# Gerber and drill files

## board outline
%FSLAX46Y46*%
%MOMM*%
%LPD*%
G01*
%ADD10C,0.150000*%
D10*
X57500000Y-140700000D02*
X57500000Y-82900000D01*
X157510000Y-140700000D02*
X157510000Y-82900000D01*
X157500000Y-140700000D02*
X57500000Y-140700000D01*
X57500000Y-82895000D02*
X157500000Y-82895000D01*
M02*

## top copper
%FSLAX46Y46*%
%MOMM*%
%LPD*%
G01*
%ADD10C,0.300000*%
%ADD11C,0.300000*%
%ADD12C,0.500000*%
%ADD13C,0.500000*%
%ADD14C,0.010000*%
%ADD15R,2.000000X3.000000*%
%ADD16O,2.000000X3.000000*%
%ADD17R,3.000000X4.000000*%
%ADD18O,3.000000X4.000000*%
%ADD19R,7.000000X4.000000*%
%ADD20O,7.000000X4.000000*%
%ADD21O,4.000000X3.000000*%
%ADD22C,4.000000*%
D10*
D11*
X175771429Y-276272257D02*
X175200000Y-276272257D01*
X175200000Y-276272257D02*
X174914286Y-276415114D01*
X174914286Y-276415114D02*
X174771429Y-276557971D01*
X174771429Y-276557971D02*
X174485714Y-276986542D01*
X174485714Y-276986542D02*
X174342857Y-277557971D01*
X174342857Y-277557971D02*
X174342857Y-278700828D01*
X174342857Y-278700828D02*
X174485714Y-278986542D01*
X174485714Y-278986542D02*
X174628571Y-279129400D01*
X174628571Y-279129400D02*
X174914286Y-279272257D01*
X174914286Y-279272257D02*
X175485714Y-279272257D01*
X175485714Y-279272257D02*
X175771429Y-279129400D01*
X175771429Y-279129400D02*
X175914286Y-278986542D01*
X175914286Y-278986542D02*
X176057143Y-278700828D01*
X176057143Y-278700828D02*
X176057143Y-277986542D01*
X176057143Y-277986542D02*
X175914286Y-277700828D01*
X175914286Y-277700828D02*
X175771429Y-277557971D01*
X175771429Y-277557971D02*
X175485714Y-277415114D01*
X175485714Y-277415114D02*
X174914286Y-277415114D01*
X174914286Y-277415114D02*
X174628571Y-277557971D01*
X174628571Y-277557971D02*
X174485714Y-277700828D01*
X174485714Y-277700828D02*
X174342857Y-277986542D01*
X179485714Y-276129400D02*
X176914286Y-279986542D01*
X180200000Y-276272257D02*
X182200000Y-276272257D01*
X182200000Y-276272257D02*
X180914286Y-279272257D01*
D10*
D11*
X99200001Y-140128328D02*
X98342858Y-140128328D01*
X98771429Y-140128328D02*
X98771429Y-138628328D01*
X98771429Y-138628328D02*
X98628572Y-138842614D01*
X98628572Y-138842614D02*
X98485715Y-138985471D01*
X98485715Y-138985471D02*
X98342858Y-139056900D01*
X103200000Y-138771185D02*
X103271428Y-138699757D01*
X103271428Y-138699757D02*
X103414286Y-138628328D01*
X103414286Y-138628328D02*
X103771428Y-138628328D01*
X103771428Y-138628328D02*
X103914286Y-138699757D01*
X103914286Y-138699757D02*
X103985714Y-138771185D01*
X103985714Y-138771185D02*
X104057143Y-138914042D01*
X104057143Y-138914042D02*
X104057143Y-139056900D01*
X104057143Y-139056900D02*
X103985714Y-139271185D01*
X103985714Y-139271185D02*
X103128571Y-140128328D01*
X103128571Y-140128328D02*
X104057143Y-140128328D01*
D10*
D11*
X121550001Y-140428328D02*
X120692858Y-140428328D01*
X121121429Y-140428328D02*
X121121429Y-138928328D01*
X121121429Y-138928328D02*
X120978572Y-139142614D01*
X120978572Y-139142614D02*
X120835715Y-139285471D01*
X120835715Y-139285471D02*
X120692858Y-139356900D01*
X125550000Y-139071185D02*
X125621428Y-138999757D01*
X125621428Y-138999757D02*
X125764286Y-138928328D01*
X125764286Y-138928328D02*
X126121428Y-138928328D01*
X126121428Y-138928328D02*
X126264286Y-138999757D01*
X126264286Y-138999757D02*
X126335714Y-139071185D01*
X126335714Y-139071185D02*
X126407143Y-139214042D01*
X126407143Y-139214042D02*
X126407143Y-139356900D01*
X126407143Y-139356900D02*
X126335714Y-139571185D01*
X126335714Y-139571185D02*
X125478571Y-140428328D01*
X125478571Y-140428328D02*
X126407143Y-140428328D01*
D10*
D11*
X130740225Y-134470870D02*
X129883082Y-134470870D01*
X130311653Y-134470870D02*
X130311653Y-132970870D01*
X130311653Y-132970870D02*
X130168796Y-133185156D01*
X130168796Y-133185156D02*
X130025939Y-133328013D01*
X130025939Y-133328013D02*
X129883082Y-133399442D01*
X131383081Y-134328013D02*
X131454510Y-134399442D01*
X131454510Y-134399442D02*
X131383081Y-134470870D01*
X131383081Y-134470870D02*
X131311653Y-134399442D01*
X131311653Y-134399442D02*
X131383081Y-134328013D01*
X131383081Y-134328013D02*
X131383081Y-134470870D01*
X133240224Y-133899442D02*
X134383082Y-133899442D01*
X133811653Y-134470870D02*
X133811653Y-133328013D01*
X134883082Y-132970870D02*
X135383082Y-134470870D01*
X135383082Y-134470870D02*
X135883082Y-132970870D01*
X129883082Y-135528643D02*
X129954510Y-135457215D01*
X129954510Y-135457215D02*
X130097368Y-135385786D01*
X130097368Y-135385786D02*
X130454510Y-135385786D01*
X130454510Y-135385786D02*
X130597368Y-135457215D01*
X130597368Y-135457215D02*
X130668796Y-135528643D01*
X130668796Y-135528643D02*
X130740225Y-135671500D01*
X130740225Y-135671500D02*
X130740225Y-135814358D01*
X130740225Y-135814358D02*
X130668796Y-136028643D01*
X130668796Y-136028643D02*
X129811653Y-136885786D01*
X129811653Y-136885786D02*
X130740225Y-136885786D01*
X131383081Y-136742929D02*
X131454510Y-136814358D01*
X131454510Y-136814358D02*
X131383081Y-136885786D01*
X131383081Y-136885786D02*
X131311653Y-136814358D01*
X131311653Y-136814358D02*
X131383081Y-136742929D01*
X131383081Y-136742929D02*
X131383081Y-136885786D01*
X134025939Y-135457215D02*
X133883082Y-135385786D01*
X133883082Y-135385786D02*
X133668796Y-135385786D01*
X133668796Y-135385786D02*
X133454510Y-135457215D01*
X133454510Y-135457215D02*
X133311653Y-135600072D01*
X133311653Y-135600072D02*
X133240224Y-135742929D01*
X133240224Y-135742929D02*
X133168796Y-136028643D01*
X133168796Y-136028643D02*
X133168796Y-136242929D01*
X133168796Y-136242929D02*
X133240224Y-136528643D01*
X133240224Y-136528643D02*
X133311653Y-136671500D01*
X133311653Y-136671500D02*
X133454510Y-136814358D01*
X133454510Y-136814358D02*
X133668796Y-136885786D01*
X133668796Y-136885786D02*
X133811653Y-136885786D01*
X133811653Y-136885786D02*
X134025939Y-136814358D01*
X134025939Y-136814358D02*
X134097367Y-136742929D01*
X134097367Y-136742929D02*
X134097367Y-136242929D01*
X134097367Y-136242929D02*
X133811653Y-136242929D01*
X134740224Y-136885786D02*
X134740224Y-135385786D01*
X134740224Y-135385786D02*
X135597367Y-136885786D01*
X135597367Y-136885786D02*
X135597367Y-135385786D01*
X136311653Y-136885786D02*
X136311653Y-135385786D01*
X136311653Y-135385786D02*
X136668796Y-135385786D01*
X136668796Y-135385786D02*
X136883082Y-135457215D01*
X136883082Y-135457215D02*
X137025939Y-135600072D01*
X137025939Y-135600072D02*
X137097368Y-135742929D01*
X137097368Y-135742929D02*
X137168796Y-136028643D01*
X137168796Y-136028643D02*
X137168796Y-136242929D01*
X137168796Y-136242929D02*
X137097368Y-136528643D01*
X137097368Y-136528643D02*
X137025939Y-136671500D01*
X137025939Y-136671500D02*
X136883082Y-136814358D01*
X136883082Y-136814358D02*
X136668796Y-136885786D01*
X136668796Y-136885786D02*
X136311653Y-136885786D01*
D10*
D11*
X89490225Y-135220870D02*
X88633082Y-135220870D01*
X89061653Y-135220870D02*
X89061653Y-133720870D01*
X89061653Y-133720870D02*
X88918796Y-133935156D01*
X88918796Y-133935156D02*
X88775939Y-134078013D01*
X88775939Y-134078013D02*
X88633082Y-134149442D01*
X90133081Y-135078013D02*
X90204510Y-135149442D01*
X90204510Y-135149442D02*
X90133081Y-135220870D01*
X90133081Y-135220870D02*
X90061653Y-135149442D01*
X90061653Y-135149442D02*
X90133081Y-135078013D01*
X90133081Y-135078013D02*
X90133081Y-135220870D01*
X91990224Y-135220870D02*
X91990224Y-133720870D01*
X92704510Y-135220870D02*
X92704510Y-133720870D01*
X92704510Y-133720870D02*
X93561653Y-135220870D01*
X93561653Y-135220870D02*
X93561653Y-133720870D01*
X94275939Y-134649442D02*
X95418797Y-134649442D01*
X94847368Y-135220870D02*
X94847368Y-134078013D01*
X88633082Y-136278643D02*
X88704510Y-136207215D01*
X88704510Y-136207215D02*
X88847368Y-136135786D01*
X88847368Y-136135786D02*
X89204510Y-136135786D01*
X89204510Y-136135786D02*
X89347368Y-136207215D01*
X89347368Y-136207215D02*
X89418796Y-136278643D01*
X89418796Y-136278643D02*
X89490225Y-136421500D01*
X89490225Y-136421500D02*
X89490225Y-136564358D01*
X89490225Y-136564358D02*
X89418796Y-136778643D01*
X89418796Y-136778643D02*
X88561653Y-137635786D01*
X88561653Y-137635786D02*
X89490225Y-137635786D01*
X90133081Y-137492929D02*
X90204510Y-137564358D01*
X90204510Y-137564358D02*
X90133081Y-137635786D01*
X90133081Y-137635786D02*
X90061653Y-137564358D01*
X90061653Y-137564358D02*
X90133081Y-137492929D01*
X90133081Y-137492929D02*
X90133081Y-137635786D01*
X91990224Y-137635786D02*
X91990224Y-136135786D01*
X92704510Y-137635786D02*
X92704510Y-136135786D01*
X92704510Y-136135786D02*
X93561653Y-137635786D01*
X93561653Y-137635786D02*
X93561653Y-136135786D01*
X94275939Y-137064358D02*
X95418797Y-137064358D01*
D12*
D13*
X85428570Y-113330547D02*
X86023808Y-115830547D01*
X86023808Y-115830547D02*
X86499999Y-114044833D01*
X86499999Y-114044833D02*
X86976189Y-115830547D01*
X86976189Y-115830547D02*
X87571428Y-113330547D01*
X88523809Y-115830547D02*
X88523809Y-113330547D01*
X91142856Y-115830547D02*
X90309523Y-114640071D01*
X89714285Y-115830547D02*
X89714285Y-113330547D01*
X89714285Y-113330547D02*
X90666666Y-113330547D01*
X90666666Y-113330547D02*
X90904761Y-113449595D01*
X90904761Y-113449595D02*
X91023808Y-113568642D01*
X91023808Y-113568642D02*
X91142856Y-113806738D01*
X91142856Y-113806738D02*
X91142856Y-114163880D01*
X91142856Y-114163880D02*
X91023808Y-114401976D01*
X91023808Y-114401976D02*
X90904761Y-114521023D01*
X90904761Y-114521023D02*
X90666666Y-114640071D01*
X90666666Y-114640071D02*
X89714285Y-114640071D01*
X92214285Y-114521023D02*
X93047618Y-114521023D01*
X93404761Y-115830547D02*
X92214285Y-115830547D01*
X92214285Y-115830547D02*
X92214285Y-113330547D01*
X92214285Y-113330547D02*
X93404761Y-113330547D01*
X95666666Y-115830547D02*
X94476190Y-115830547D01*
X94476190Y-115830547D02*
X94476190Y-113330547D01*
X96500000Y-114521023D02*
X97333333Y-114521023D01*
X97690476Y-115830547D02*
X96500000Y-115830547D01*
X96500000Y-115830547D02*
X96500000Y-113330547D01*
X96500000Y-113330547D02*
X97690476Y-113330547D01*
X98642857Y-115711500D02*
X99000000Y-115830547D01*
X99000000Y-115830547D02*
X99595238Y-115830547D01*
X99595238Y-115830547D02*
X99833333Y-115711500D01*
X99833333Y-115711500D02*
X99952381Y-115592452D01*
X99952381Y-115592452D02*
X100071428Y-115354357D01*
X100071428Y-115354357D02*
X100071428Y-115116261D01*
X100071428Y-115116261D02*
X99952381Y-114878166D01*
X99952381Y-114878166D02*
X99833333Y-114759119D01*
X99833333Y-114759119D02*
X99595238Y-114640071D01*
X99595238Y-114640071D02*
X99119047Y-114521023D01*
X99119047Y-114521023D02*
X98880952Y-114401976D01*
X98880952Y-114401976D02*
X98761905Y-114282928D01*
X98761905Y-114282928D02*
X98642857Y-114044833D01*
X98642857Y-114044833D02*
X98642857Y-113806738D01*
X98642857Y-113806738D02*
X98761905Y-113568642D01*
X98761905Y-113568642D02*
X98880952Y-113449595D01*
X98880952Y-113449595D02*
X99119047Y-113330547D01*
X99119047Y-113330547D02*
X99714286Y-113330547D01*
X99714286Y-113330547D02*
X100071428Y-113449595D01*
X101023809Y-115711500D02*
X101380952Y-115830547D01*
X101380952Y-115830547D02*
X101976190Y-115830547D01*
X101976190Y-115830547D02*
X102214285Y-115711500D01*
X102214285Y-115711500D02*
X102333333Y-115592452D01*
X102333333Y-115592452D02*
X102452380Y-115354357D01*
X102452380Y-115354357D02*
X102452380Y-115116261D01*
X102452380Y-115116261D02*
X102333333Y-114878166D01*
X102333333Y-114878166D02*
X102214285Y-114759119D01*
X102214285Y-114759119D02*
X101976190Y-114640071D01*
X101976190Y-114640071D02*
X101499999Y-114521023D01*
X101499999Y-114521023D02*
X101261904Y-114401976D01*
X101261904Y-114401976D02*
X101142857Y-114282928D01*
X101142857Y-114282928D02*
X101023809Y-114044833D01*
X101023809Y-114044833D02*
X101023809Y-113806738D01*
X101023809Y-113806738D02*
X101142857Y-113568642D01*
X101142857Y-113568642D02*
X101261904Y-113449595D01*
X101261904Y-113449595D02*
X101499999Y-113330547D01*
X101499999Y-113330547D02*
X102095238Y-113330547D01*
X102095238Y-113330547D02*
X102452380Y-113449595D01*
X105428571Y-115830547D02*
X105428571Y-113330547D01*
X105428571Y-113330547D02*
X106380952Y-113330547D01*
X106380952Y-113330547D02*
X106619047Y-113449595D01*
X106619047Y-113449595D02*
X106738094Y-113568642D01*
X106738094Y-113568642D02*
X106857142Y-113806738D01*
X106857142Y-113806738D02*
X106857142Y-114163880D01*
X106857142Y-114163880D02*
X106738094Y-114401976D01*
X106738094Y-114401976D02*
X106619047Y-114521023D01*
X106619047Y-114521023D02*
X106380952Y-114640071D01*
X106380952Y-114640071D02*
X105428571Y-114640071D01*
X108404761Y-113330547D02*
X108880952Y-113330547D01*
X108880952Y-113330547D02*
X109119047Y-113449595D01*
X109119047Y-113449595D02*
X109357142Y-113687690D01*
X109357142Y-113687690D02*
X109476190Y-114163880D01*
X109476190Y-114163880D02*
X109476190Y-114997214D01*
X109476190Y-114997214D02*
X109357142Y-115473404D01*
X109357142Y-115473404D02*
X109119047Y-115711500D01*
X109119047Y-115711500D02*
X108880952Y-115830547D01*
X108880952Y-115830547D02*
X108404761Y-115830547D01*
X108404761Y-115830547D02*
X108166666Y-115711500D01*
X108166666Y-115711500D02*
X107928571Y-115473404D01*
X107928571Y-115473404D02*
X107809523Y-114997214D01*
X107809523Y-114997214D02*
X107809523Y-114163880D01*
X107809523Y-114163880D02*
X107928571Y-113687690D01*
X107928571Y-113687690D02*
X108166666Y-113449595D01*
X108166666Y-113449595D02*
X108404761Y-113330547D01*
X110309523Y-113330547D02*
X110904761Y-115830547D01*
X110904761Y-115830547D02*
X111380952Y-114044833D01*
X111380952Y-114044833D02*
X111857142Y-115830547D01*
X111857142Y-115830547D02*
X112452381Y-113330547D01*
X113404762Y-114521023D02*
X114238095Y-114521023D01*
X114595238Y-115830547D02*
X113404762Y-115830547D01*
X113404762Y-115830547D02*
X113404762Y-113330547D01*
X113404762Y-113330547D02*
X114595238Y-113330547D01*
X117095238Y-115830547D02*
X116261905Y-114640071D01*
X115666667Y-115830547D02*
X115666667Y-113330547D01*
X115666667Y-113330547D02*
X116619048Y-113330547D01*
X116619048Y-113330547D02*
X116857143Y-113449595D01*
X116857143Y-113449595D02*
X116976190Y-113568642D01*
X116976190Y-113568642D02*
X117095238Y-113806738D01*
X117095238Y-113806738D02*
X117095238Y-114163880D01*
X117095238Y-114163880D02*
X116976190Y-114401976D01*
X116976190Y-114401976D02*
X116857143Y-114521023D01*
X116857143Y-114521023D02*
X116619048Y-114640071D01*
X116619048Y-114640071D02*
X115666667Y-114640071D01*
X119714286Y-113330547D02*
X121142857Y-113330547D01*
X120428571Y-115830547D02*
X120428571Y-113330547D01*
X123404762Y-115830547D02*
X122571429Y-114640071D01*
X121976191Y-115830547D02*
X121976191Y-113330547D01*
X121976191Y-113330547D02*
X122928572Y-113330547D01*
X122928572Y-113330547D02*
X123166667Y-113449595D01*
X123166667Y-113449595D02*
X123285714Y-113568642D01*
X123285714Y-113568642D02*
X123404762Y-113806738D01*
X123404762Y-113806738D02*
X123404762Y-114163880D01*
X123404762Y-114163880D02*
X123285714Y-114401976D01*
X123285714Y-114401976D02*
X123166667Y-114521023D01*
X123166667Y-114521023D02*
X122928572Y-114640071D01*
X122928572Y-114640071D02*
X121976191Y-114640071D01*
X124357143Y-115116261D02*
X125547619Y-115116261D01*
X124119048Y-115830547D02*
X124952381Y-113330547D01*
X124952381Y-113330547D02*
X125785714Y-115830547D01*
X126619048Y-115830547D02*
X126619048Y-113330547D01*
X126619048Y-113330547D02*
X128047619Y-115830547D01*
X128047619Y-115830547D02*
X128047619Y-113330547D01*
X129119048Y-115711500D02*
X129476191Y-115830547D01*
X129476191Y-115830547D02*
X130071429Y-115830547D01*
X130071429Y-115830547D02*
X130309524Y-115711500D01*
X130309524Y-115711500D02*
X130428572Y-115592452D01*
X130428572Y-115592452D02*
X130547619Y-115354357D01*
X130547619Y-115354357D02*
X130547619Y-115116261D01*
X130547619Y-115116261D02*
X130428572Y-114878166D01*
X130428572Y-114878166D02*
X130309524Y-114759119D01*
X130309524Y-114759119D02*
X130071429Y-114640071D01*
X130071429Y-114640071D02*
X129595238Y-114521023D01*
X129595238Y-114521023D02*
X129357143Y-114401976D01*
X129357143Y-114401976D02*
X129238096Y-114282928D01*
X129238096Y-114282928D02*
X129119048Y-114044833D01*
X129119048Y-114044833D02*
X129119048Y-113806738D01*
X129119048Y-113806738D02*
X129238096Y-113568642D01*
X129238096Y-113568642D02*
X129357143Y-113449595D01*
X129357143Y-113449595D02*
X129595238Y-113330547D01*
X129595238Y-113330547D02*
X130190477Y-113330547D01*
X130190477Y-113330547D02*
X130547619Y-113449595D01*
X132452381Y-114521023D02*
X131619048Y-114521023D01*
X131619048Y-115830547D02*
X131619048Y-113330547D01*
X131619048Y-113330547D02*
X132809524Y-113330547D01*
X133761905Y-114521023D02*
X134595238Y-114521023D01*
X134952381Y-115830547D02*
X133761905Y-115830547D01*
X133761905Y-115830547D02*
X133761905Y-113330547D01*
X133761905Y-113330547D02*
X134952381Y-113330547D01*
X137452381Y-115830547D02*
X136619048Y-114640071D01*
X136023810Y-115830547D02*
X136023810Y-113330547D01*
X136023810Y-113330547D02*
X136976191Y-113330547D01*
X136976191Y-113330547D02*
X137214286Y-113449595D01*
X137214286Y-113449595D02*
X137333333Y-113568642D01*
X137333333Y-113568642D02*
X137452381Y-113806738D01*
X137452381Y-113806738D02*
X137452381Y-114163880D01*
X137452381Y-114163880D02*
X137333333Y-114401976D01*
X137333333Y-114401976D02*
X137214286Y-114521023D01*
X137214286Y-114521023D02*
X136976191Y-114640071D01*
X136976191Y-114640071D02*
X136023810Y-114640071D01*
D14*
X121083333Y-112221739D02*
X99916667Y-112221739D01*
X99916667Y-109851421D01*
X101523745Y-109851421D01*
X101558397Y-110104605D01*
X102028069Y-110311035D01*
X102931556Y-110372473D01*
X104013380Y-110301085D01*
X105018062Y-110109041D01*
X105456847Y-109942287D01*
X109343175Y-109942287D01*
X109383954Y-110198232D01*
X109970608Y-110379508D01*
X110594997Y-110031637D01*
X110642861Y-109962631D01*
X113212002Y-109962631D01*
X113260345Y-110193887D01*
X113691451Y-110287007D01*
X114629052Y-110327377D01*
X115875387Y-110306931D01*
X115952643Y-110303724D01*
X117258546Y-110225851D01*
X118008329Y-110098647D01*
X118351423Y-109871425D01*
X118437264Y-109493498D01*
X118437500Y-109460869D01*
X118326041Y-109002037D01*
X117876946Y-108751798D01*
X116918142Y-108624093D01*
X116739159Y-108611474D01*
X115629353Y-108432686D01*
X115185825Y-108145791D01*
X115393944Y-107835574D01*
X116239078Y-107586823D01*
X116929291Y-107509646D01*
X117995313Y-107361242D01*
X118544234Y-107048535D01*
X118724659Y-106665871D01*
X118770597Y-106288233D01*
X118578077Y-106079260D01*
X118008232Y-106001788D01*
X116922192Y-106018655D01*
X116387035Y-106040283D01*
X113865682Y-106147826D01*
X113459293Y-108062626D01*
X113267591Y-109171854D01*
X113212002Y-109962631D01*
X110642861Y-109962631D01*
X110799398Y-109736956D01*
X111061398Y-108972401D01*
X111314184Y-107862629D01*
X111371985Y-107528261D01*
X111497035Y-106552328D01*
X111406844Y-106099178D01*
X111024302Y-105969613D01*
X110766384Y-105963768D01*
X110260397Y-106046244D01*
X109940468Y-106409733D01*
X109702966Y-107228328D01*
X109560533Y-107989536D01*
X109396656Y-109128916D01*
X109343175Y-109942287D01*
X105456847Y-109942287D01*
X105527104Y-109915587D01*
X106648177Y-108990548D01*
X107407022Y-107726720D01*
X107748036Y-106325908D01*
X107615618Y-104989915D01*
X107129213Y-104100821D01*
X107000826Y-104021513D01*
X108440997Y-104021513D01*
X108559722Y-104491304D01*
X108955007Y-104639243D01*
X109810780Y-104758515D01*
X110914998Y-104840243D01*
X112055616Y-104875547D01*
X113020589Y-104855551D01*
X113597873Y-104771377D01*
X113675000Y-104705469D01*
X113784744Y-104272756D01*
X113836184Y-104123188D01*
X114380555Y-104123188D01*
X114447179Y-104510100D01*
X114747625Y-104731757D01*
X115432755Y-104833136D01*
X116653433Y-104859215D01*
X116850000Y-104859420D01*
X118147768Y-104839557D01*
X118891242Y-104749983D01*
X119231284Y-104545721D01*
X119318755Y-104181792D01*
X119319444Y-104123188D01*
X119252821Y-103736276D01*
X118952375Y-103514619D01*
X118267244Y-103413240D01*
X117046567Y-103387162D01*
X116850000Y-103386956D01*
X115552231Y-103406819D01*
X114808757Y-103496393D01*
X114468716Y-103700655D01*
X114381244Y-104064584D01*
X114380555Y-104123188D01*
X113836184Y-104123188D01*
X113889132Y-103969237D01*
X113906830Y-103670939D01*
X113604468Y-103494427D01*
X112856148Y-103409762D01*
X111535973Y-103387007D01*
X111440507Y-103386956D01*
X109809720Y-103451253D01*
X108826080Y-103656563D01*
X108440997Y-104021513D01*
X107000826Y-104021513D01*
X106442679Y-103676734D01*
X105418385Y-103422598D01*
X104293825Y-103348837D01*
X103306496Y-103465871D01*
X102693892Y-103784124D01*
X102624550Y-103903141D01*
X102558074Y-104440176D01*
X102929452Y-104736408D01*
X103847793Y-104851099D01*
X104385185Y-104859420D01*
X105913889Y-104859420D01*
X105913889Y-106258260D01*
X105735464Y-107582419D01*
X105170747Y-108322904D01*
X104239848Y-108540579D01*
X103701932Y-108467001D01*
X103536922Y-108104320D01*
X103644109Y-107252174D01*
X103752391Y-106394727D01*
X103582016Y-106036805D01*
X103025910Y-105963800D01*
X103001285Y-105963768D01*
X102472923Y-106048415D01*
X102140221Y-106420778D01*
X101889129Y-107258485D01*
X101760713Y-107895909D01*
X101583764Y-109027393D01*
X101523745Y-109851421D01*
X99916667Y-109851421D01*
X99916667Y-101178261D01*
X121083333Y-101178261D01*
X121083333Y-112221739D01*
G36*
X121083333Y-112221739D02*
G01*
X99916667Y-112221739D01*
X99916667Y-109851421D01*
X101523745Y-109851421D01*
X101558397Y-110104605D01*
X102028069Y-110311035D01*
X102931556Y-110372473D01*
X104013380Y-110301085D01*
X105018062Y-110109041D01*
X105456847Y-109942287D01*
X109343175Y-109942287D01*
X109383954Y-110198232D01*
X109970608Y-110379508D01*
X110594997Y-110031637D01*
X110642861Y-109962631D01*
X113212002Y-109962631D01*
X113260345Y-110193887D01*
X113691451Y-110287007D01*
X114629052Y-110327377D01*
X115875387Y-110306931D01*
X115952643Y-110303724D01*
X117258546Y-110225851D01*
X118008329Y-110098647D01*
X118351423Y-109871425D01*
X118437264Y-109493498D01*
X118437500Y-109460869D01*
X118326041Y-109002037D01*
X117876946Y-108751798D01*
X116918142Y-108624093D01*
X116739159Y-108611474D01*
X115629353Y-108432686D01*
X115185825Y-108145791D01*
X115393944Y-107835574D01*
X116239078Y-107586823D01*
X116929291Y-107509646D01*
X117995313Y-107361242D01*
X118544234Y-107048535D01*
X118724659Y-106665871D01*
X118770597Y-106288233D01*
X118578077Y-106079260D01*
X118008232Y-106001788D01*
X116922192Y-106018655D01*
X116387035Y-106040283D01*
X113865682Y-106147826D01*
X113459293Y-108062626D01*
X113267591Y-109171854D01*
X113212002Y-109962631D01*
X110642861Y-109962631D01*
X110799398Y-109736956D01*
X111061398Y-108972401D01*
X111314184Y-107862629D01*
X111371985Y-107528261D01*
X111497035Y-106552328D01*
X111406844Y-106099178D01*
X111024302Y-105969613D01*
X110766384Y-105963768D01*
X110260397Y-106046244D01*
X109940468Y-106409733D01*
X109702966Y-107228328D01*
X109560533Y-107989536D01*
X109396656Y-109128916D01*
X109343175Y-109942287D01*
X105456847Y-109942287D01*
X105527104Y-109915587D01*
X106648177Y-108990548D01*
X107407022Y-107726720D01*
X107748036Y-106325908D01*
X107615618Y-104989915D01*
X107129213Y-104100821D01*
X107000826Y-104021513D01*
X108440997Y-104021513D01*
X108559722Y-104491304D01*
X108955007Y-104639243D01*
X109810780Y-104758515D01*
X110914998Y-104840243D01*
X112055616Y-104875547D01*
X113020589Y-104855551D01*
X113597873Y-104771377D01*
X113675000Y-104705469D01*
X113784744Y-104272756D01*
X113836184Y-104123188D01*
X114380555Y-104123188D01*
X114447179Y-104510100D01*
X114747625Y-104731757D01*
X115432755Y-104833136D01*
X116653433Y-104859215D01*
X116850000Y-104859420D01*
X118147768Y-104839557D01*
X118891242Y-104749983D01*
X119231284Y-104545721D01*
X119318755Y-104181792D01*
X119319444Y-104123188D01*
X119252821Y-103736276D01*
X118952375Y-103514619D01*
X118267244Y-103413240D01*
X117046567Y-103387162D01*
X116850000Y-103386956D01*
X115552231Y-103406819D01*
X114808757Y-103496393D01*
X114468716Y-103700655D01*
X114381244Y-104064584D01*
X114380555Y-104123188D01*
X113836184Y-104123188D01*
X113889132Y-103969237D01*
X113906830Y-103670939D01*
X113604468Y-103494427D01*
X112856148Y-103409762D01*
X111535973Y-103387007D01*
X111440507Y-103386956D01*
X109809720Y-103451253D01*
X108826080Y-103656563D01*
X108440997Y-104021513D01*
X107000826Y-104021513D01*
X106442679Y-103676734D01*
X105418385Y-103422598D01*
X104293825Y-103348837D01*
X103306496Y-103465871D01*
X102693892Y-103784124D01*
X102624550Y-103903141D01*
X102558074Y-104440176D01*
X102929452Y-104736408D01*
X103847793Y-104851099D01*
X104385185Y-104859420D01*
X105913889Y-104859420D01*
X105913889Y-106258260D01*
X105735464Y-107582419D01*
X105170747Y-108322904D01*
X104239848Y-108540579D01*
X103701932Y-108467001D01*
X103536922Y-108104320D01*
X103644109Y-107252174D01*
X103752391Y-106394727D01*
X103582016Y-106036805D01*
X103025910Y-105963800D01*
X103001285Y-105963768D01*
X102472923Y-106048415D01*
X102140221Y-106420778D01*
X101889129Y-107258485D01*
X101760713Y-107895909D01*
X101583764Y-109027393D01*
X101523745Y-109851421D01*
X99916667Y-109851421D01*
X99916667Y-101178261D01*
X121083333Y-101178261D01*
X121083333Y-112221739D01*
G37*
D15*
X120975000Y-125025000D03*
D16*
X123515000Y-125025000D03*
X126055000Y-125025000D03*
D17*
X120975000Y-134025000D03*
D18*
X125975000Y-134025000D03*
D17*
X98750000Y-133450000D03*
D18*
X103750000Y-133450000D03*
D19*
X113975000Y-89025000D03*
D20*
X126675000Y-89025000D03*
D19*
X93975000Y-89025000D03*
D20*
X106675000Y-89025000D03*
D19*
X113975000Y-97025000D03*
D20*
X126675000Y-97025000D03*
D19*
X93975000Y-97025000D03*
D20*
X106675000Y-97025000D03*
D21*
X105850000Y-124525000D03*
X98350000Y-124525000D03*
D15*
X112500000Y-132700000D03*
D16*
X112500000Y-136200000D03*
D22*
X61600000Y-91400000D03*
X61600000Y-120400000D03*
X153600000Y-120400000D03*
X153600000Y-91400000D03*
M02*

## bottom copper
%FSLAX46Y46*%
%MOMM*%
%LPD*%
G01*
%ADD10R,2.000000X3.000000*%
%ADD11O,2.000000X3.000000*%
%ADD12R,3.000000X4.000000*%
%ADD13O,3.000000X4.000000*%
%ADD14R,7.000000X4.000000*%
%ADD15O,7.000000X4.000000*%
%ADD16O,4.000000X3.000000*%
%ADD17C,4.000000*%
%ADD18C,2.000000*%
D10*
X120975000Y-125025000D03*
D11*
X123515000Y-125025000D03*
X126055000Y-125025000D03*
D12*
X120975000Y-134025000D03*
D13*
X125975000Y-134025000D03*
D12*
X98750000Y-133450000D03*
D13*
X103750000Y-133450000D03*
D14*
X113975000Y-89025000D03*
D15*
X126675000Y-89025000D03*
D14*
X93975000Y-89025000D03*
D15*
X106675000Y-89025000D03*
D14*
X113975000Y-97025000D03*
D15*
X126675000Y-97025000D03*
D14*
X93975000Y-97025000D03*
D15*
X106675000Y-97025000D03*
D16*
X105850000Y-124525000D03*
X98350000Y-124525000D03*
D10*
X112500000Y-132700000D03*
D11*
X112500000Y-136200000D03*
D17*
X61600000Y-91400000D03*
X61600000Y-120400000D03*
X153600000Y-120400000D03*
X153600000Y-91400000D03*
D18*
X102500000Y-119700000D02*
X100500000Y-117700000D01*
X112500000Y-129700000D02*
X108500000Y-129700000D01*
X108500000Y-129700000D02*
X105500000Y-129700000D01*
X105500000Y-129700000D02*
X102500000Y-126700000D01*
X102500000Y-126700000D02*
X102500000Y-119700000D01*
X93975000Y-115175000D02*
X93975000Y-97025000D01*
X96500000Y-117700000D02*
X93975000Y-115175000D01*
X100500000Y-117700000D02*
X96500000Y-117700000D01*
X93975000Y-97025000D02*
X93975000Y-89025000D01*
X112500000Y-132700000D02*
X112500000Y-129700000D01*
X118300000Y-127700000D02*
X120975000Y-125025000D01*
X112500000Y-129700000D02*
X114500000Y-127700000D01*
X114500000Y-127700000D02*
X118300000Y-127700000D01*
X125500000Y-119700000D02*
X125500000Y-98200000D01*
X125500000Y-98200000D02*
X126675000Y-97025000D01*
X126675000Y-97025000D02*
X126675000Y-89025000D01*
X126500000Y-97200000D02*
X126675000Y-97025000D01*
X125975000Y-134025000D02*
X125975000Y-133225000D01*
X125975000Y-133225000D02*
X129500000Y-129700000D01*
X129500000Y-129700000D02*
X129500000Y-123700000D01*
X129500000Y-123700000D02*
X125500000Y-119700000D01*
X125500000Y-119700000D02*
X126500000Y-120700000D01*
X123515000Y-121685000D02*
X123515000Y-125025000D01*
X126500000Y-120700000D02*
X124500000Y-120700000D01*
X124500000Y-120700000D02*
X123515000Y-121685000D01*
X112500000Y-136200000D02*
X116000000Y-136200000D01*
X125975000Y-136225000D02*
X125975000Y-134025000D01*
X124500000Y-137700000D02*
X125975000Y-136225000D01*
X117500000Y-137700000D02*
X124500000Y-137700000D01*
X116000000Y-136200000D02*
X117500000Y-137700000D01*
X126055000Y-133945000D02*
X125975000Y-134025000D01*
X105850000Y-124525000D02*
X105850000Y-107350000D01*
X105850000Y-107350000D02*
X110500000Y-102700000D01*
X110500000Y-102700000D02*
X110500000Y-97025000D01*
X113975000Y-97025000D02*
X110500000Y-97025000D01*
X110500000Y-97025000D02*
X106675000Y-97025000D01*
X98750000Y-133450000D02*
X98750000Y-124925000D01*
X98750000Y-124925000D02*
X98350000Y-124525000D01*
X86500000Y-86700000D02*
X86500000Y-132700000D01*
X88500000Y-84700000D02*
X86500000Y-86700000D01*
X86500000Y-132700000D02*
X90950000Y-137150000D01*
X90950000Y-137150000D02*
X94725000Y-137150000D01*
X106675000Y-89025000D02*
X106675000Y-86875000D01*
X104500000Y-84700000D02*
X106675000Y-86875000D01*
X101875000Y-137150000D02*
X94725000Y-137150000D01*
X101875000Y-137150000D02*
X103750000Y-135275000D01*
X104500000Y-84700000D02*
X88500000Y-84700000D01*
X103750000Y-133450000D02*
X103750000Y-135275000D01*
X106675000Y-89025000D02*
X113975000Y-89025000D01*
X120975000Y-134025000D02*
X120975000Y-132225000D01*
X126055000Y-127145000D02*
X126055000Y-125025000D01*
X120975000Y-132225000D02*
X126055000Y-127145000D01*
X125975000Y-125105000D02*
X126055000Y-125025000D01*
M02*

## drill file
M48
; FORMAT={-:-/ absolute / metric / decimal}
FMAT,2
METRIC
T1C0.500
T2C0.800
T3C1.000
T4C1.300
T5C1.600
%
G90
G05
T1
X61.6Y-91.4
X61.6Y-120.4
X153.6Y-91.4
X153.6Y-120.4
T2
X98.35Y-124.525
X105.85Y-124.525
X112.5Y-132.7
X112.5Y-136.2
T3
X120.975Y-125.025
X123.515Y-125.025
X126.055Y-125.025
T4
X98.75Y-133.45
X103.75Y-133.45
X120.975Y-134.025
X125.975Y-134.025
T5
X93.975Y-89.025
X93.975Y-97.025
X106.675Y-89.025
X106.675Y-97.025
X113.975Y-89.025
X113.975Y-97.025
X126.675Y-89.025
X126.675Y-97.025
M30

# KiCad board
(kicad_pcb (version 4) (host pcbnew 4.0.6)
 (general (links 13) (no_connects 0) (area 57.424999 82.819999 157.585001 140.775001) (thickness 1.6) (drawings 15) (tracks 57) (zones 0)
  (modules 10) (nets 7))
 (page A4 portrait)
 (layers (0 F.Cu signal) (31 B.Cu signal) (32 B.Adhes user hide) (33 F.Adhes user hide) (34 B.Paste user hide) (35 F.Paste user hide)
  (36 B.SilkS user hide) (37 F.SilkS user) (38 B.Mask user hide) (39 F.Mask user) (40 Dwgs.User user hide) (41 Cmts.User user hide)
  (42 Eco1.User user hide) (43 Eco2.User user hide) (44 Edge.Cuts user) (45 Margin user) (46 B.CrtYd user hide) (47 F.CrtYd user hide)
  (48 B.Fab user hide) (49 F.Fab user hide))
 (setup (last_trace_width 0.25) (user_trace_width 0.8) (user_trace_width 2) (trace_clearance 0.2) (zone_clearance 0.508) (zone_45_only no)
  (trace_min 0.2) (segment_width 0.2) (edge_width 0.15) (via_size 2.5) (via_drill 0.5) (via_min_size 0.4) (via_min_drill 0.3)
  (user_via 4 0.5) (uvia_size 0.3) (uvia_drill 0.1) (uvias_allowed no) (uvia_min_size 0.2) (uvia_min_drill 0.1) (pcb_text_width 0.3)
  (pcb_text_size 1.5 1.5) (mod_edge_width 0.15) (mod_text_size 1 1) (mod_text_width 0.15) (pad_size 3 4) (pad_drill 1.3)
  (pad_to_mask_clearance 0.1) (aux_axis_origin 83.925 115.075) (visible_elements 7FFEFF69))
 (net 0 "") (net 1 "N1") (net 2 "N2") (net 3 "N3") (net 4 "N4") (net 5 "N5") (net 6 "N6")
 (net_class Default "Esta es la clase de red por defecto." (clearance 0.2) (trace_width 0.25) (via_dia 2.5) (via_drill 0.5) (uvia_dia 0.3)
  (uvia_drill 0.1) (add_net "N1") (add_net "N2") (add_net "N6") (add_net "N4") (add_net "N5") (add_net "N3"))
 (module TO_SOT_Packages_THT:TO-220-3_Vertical (layer F.Cu) (at 120.975 125.025)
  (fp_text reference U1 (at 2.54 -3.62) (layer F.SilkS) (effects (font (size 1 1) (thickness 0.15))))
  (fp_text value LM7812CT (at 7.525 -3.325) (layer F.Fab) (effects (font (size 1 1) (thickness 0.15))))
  (pad 1 thru_hole rect (at 0 0) (size 2 3) (drill 1) (layers *.Cu *.Mask) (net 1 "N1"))
  (pad 2 thru_hole oval (at 2.54 0) (size 2 3) (drill 1) (layers *.Cu *.Mask) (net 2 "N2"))
  (pad 3 thru_hole oval (at 5.08 0) (size 2 3) (drill 1) (layers *.Cu *.Mask) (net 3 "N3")))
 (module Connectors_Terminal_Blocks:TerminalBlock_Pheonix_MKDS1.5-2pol (layer F.Cu) (at 120.975 134.025)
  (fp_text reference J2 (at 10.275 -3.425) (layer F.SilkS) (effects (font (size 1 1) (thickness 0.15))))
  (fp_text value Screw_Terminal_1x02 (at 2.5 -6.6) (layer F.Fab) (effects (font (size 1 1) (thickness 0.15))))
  (pad 1 thru_hole rect (at 0 0) (size 3 4) (drill 1.3) (layers *.Cu *.Mask) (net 3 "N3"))
  (pad 2 thru_hole oval (at 5 0) (size 3 4) (drill 1.3) (layers *.Cu *.Mask) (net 2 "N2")))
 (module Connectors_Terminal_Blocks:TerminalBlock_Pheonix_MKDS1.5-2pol (layer F.Cu) (at 98.75 133.45)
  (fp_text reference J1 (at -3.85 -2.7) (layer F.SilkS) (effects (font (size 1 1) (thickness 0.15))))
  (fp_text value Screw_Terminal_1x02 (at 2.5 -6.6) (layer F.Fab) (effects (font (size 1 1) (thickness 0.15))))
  (pad 1 thru_hole rect (at 0 0) (size 3 4) (drill 1.3) (layers *.Cu *.Mask) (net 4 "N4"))
  (pad 2 thru_hole oval (at 5 0) (size 3 4) (drill 1.3) (layers *.Cu *.Mask) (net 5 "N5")))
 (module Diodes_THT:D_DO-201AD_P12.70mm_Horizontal (layer F.Cu) (at 113.975 89.025)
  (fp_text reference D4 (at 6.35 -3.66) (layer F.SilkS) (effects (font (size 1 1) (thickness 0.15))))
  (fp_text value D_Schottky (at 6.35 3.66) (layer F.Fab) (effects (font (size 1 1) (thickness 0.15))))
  (pad 1 thru_hole rect (at 0 0) (size 7 4) (drill 1.6) (layers *.Cu *.Mask) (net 5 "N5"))
  (pad 2 thru_hole oval (at 12.7 0) (size 7 4) (drill 1.6) (layers *.Cu *.Mask) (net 2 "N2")))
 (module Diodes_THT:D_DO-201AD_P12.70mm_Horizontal (layer F.Cu) (at 93.975 89.025)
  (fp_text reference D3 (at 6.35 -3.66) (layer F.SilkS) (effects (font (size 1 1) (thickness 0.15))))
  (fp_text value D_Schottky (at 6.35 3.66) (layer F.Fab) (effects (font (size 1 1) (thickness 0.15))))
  (pad 1 thru_hole rect (at 0 0) (size 7 4) (drill 1.6) (layers *.Cu *.Mask) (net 1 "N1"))
  (pad 2 thru_hole oval (at 12.7 0) (size 7 4) (drill 1.6) (layers *.Cu *.Mask) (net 5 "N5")))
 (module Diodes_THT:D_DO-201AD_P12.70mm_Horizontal (layer F.Cu) (at 113.975 97.025)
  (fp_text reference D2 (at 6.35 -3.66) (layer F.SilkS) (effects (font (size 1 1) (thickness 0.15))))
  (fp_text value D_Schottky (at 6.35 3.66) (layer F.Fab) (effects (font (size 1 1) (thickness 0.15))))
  (pad 1 thru_hole rect (at 0 0) (size 7 4) (drill 1.6) (layers *.Cu *.Mask) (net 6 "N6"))
  (pad 2 thru_hole oval (at 12.7 0) (size 7 4) (drill 1.6) (layers *.Cu *.Mask) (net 2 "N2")))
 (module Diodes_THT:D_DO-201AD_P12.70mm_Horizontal (layer F.Cu) (at 93.975 97.025)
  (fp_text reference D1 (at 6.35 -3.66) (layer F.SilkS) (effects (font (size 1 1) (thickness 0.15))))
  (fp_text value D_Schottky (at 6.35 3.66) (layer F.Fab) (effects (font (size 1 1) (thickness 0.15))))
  (pad 1 thru_hole rect (at 0 0) (size 7 4) (drill 1.6) (layers *.Cu *.Mask) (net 1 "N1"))
  (pad 2 thru_hole oval (at 12.7 0) (size 7 4) (drill 1.6) (layers *.Cu *.Mask) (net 6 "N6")))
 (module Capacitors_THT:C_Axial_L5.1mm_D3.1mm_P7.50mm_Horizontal (layer F.Cu) (at 105.85 124.525 180)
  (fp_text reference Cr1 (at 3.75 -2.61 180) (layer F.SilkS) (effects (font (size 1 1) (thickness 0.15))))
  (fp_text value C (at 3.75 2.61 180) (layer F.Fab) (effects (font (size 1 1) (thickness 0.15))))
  (pad 1 thru_hole oval (at 0 0 180) (size 4 3) (drill 0.8) (layers *.Cu *.Mask) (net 6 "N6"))
  (pad 2 thru_hole oval (at 7.5 0 180) (size 4 3) (drill 0.8) (layers *.Cu *.Mask) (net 4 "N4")))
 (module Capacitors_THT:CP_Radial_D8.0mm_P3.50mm (layer F.Cu) (at 112.5 132.7 270)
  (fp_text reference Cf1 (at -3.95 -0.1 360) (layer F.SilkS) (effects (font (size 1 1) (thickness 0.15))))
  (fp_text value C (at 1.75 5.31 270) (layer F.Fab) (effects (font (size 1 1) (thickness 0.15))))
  (pad 1 thru_hole rect (at 0 0 270) (size 3 2) (drill 0.8) (layers *.Cu *.Mask) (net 1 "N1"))
  (pad 2 thru_hole oval (at 3.5 0 270) (size 3 2) (drill 0.8) (layers *.Cu *.Mask) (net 2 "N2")))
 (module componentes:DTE (layer F.Cu) (at 110.5 106.7)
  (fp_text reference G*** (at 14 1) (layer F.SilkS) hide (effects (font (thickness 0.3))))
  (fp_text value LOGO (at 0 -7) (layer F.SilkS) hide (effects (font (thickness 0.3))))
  (fp_poly
   (pts (xy 10.583333 5.521739) (xy -10.583333 5.521739) (xy -10.583333 3.151421) (xy -8.976255 3.151421) (xy -8.941603 3.404605)
    (xy -8.471931 3.611035) (xy -7.568444 3.672473) (xy -6.48662 3.601085) (xy -5.481938 3.409041) (xy -5.043153 3.242287)
    (xy -1.156825 3.242287) (xy -1.116046 3.498232) (xy -0.529392 3.679508) (xy 0.094997 3.331637) (xy 0.142861 3.262631)
    (xy 2.712002 3.262631) (xy 2.760345 3.493887) (xy 3.191451 3.587007) (xy 4.129052 3.627377) (xy 5.375387 3.606931)
    (xy 5.452643 3.603724) (xy 6.758546 3.525851) (xy 7.508329 3.398647) (xy 7.851423 3.171425) (xy 7.937264 2.793498) (xy 7.9375 2.760869)
    (xy 7.826041 2.302037) (xy 7.376946 2.051798) (xy 6.418142 1.924093) (xy 6.239159 1.911474) (xy 5.129353 1.732686)
    (xy 4.685825 1.445791) (xy 4.893944 1.135574) (xy 5.739078 0.886823) (xy 6.429291 0.809646) (xy 7.495313 0.661242)
    (xy 8.044234 0.348535) (xy 8.224659 -0.034129) (xy 8.270597 -0.411767) (xy 8.078077 -0.62074) (xy 7.508232 -0.698212)
    (xy 6.422192 -0.681345) (xy 5.887035 -0.659717) (xy 3.365682 -0.552174) (xy 2.959293 1.362626) (xy 2.767591 2.471854)
    (xy 2.712002 3.262631) (xy 0.142861 3.262631) (xy 0.299398 3.036956) (xy 0.561398 2.272401) (xy 0.814184 1.162629)
    (xy 0.871985 0.828261) (xy 0.997035 -0.147672) (xy 0.906844 -0.600822) (xy 0.524302 -0.730387) (xy 0.266384 -0.736232)
    (xy -0.239603 -0.653756) (xy -0.559532 -0.290267) (xy -0.797034 0.528328) (xy -0.939467 1.289536) (xy -1.103344 2.428916)
    (xy -1.156825 3.242287) (xy -5.043153 3.242287) (xy -4.972896 3.215587) (xy -3.851823 2.290548) (xy -3.092978 1.02672)
    (xy -2.751964 -0.374092) (xy -2.884382 -1.710085) (xy -3.370787 -2.599179) (xy -3.499174 -2.678487) (xy -2.059003 -2.678487)
    (xy -1.940278 -2.208696) (xy -1.544993 -2.060757) (xy -0.68922 -1.941485) (xy 0.414998 -1.859757) (xy 1.555616 -1.824453)
    (xy 2.520589 -1.844449) (xy 3.097873 -1.928623) (xy 3.175 -1.994531) (xy 3.284744 -2.427244) (xy 3.336184 -2.576812)
    (xy 3.880555 -2.576812) (xy 3.947179 -2.1899) (xy 4.247625 -1.968243) (xy 4.932755 -1.866864) (xy 6.153433 -1.840785) (xy 6.35 -1.84058)
    (xy 7.647768 -1.860443) (xy 8.391242 -1.950017) (xy 8.731284 -2.154279) (xy 8.818755 -2.518208) (xy 8.819444 -2.576812)
    (xy 8.752821 -2.963724) (xy 8.452375 -3.185381) (xy 7.767244 -3.28676) (xy 6.546567 -3.312838) (xy 6.35 -3.313044)
    (xy 5.052231 -3.293181) (xy 4.308757 -3.203607) (xy 3.968716 -2.999345) (xy 3.881244 -2.635416) (xy 3.880555 -2.576812)
    (xy 3.336184 -2.576812) (xy 3.389132 -2.730763) (xy 3.40683 -3.029061) (xy 3.104468 -3.205573) (xy 2.356148 -3.290238)
    (xy 1.035973 -3.312993) (xy 0.940507 -3.313044) (xy -0.69028 -3.248747) (xy -1.67392 -3.043437) (xy -2.059003 -2.678487)
    (xy -3.499174 -2.678487) (xy -4.057321 -3.023266) (xy -5.081615 -3.277402) (xy -6.206175 -3.351163) (xy -7.193504 -3.234129)
    (xy -7.806108 -2.915876) (xy -7.87545 -2.796859) (xy -7.941926 -2.259824) (xy -7.570548 -1.963592) (xy -6.652207 -1.848901)
    (xy -6.114815 -1.84058) (xy -4.586111 -1.84058) (xy -4.586111 -0.44174) (xy -4.764536 0.882419) (xy -5.329253 1.622904)
    (xy -6.260152 1.840579) (xy -6.798068 1.767001) (xy -6.963078 1.40432) (xy -6.855891 0.552174) (xy -6.747609 -0.305273)
    (xy -6.917984 -0.663195) (xy -7.47409 -0.7362) (xy -7.498715 -0.736232) (xy -8.027077 -0.651585) (xy -8.359779 -0.279222)
    (xy -8.610871 0.558485) (xy -8.739287 1.195909) (xy -8.916236 2.327393) (xy -8.976255 3.151421) (xy -10.583333 3.151421)
    (xy -10.583333 -5.521739) (xy 10.583333 -5.521739) (xy 10.583333 5.521739))
   (layer F.Cu) (width 0.01)))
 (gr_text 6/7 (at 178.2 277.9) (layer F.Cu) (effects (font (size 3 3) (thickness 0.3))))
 (gr_line (start 57.5 140.7) (end 57.5 82.9) (angle 90) (layer Edge.Cuts) (width 0.15))
 (gr_line (start 157.51 140.7) (end 157.51 82.9) (angle 90) (layer Edge.Cuts) (width 0.15))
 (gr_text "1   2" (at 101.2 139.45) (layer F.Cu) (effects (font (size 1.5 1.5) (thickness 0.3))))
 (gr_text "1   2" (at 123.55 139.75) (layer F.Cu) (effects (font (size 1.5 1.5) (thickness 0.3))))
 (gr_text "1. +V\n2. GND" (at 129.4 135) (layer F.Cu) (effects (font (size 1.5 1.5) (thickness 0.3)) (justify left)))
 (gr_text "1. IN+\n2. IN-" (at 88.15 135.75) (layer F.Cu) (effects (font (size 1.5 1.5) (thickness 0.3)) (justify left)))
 (gr_line (start 157.5 140.7) (end 57.5 140.7) (angle 90) (layer Edge.Cuts) (width 0.15))
 (gr_line (start 57.5 82.895) (end 157.5 82.895) (angle 90) (layer Edge.Cuts) (width 0.15))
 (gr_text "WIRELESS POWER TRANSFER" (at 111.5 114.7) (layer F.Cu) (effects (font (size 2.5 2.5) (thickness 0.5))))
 (via (at 61.6 91.4) (size 4) (drill 0.5) (layers F.Cu B.Cu) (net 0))
 (via (at 61.6 120.4) (size 4) (drill 0.5) (layers F.Cu B.Cu) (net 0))
 (via (at 153.6 120.4) (size 4) (drill 0.5) (layers F.Cu B.Cu) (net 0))
 (via (at 153.6 91.4) (size 4) (drill 0.5) (layers F.Cu B.Cu) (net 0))
 (segment (start 102.5 119.7) (end 100.5 117.7) (width 2) (layer B.Cu) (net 1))
 (segment (start 112.5 129.7) (end 108.5 129.7) (width 2) (layer B.Cu) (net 1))
 (segment (start 108.5 129.7) (end 105.5 129.7) (width 2) (layer B.Cu) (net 1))
 (segment (start 105.5 129.7) (end 102.5 126.7) (width 2) (layer B.Cu) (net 1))
 (segment (start 102.5 126.7) (end 102.5 119.7) (width 2) (layer B.Cu) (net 1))
 (segment (start 93.975 115.175) (end 93.975 97.025) (width 2) (layer B.Cu) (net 1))
 (segment (start 96.5 117.7) (end 93.975 115.175) (width 2) (layer B.Cu) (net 1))
 (segment (start 100.5 117.7) (end 96.5 117.7) (width 2) (layer B.Cu) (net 1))
 (segment (start 93.975 97.025) (end 93.975 89.025) (width 2) (layer B.Cu) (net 1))
 (segment (start 112.5 132.7) (end 112.5 129.7) (width 2) (layer B.Cu) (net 1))
 (segment (start 118.3 127.7) (end 120.975 125.025) (width 2) (layer B.Cu) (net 1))
 (segment (start 112.5 129.7) (end 114.5 127.7) (width 2) (layer B.Cu) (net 1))
 (segment (start 114.5 127.7) (end 118.3 127.7) (width 2) (layer B.Cu) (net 1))
 (segment (start 125.5 119.7) (end 125.5 98.2) (width 2) (layer B.Cu) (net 2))
 (segment (start 125.5 98.2) (end 126.675 97.025) (width 2) (layer B.Cu) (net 2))
 (segment (start 126.675 97.025) (end 126.675 89.025) (width 2) (layer B.Cu) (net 2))
 (segment (start 126.5 97.2) (end 126.675 97.025) (width 2) (layer B.Cu) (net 2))
 (segment (start 125.975 134.025) (end 125.975 133.225) (width 2) (layer B.Cu) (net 2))
 (segment (start 125.975 133.225) (end 129.5 129.7) (width 2) (layer B.Cu) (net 2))
 (segment (start 129.5 129.7) (end 129.5 123.7) (width 2) (layer B.Cu) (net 2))
 (segment (start 129.5 123.7) (end 125.5 119.7) (width 2) (layer B.Cu) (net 2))
 (segment (start 125.5 119.7) (end 126.5 120.7) (width 2) (layer B.Cu) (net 2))
 (segment (start 123.515 121.685) (end 123.515 125.025) (width 2) (layer B.Cu) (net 2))
 (segment (start 126.5 120.7) (end 124.5 120.7) (width 2) (layer B.Cu) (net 2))
 (segment (start 124.5 120.7) (end 123.515 121.685) (width 2) (layer B.Cu) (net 2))
 (segment (start 112.5 136.2) (end 116 136.2) (width 2) (layer B.Cu) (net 2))
 (segment (start 125.975 136.225) (end 125.975 134.025) (width 2) (layer B.Cu) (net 2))
 (segment (start 124.5 137.7) (end 125.975 136.225) (width 2) (layer B.Cu) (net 2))
 (segment (start 117.5 137.7) (end 124.5 137.7) (width 2) (layer B.Cu) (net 2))
 (segment (start 116 136.2) (end 117.5 137.7) (width 2) (layer B.Cu) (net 2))
 (segment (start 126.055 133.945) (end 125.975 134.025) (width 2) (layer B.Cu) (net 2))
 (segment (start 105.85 124.525) (end 105.85 107.35) (width 2) (layer B.Cu) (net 6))
 (segment (start 105.85 107.35) (end 110.5 102.7) (width 2) (layer B.Cu) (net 6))
 (segment (start 110.5 102.7) (end 110.5 97.025) (width 2) (layer B.Cu) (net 6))
 (segment (start 113.975 97.025) (end 110.5 97.025) (width 2) (layer B.Cu) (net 6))
 (segment (start 110.5 97.025) (end 106.675 97.025) (width 2) (layer B.Cu) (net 6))
 (segment (start 98.75 133.45) (end 98.75 124.925) (width 2) (layer B.Cu) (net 4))
 (segment (start 98.75 124.925) (end 98.35 124.525) (width 2) (layer B.Cu) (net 4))
 (segment (start 86.5 86.7) (end 86.5 132.7) (width 2) (layer B.Cu) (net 5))
 (segment (start 88.5 84.7) (end 86.5 86.7) (width 2) (layer B.Cu) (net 5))
 (segment (start 86.5 132.7) (end 90.95 137.15) (width 2) (layer B.Cu) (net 5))
 (segment (start 90.95 137.15) (end 94.725 137.15) (width 2) (layer B.Cu) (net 5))
 (segment (start 106.675 89.025) (end 106.675 86.875) (width 2) (layer B.Cu) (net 5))
 (segment (start 104.5 84.7) (end 106.675 86.875) (width 2) (layer B.Cu) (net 5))
 (segment (start 101.875 137.15) (end 94.725 137.15) (width 2) (layer B.Cu) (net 5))
 (segment (start 101.875 137.15) (end 103.75 135.275) (width 2) (layer B.Cu) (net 5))
 (segment (start 104.5 84.7) (end 88.5 84.7) (width 2) (layer B.Cu) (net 5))
 (segment (start 103.75 133.45) (end 103.75 135.275) (width 2) (layer B.Cu) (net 5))
 (segment (start 106.675 89.025) (end 113.975 89.025) (width 2) (layer B.Cu) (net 5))
 (segment (start 120.975 134.025) (end 120.975 132.225) (width 2) (layer B.Cu) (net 3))
 (segment (start 126.055 127.145) (end 126.055 125.025) (width 2) (layer B.Cu) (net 3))
 (segment (start 120.975 132.225) (end 126.055 127.145) (width 2) (layer B.Cu) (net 3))
 (segment (start 125.975 125.105) (end 126.055 125.025) (width 2) (layer B.Cu) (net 3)))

